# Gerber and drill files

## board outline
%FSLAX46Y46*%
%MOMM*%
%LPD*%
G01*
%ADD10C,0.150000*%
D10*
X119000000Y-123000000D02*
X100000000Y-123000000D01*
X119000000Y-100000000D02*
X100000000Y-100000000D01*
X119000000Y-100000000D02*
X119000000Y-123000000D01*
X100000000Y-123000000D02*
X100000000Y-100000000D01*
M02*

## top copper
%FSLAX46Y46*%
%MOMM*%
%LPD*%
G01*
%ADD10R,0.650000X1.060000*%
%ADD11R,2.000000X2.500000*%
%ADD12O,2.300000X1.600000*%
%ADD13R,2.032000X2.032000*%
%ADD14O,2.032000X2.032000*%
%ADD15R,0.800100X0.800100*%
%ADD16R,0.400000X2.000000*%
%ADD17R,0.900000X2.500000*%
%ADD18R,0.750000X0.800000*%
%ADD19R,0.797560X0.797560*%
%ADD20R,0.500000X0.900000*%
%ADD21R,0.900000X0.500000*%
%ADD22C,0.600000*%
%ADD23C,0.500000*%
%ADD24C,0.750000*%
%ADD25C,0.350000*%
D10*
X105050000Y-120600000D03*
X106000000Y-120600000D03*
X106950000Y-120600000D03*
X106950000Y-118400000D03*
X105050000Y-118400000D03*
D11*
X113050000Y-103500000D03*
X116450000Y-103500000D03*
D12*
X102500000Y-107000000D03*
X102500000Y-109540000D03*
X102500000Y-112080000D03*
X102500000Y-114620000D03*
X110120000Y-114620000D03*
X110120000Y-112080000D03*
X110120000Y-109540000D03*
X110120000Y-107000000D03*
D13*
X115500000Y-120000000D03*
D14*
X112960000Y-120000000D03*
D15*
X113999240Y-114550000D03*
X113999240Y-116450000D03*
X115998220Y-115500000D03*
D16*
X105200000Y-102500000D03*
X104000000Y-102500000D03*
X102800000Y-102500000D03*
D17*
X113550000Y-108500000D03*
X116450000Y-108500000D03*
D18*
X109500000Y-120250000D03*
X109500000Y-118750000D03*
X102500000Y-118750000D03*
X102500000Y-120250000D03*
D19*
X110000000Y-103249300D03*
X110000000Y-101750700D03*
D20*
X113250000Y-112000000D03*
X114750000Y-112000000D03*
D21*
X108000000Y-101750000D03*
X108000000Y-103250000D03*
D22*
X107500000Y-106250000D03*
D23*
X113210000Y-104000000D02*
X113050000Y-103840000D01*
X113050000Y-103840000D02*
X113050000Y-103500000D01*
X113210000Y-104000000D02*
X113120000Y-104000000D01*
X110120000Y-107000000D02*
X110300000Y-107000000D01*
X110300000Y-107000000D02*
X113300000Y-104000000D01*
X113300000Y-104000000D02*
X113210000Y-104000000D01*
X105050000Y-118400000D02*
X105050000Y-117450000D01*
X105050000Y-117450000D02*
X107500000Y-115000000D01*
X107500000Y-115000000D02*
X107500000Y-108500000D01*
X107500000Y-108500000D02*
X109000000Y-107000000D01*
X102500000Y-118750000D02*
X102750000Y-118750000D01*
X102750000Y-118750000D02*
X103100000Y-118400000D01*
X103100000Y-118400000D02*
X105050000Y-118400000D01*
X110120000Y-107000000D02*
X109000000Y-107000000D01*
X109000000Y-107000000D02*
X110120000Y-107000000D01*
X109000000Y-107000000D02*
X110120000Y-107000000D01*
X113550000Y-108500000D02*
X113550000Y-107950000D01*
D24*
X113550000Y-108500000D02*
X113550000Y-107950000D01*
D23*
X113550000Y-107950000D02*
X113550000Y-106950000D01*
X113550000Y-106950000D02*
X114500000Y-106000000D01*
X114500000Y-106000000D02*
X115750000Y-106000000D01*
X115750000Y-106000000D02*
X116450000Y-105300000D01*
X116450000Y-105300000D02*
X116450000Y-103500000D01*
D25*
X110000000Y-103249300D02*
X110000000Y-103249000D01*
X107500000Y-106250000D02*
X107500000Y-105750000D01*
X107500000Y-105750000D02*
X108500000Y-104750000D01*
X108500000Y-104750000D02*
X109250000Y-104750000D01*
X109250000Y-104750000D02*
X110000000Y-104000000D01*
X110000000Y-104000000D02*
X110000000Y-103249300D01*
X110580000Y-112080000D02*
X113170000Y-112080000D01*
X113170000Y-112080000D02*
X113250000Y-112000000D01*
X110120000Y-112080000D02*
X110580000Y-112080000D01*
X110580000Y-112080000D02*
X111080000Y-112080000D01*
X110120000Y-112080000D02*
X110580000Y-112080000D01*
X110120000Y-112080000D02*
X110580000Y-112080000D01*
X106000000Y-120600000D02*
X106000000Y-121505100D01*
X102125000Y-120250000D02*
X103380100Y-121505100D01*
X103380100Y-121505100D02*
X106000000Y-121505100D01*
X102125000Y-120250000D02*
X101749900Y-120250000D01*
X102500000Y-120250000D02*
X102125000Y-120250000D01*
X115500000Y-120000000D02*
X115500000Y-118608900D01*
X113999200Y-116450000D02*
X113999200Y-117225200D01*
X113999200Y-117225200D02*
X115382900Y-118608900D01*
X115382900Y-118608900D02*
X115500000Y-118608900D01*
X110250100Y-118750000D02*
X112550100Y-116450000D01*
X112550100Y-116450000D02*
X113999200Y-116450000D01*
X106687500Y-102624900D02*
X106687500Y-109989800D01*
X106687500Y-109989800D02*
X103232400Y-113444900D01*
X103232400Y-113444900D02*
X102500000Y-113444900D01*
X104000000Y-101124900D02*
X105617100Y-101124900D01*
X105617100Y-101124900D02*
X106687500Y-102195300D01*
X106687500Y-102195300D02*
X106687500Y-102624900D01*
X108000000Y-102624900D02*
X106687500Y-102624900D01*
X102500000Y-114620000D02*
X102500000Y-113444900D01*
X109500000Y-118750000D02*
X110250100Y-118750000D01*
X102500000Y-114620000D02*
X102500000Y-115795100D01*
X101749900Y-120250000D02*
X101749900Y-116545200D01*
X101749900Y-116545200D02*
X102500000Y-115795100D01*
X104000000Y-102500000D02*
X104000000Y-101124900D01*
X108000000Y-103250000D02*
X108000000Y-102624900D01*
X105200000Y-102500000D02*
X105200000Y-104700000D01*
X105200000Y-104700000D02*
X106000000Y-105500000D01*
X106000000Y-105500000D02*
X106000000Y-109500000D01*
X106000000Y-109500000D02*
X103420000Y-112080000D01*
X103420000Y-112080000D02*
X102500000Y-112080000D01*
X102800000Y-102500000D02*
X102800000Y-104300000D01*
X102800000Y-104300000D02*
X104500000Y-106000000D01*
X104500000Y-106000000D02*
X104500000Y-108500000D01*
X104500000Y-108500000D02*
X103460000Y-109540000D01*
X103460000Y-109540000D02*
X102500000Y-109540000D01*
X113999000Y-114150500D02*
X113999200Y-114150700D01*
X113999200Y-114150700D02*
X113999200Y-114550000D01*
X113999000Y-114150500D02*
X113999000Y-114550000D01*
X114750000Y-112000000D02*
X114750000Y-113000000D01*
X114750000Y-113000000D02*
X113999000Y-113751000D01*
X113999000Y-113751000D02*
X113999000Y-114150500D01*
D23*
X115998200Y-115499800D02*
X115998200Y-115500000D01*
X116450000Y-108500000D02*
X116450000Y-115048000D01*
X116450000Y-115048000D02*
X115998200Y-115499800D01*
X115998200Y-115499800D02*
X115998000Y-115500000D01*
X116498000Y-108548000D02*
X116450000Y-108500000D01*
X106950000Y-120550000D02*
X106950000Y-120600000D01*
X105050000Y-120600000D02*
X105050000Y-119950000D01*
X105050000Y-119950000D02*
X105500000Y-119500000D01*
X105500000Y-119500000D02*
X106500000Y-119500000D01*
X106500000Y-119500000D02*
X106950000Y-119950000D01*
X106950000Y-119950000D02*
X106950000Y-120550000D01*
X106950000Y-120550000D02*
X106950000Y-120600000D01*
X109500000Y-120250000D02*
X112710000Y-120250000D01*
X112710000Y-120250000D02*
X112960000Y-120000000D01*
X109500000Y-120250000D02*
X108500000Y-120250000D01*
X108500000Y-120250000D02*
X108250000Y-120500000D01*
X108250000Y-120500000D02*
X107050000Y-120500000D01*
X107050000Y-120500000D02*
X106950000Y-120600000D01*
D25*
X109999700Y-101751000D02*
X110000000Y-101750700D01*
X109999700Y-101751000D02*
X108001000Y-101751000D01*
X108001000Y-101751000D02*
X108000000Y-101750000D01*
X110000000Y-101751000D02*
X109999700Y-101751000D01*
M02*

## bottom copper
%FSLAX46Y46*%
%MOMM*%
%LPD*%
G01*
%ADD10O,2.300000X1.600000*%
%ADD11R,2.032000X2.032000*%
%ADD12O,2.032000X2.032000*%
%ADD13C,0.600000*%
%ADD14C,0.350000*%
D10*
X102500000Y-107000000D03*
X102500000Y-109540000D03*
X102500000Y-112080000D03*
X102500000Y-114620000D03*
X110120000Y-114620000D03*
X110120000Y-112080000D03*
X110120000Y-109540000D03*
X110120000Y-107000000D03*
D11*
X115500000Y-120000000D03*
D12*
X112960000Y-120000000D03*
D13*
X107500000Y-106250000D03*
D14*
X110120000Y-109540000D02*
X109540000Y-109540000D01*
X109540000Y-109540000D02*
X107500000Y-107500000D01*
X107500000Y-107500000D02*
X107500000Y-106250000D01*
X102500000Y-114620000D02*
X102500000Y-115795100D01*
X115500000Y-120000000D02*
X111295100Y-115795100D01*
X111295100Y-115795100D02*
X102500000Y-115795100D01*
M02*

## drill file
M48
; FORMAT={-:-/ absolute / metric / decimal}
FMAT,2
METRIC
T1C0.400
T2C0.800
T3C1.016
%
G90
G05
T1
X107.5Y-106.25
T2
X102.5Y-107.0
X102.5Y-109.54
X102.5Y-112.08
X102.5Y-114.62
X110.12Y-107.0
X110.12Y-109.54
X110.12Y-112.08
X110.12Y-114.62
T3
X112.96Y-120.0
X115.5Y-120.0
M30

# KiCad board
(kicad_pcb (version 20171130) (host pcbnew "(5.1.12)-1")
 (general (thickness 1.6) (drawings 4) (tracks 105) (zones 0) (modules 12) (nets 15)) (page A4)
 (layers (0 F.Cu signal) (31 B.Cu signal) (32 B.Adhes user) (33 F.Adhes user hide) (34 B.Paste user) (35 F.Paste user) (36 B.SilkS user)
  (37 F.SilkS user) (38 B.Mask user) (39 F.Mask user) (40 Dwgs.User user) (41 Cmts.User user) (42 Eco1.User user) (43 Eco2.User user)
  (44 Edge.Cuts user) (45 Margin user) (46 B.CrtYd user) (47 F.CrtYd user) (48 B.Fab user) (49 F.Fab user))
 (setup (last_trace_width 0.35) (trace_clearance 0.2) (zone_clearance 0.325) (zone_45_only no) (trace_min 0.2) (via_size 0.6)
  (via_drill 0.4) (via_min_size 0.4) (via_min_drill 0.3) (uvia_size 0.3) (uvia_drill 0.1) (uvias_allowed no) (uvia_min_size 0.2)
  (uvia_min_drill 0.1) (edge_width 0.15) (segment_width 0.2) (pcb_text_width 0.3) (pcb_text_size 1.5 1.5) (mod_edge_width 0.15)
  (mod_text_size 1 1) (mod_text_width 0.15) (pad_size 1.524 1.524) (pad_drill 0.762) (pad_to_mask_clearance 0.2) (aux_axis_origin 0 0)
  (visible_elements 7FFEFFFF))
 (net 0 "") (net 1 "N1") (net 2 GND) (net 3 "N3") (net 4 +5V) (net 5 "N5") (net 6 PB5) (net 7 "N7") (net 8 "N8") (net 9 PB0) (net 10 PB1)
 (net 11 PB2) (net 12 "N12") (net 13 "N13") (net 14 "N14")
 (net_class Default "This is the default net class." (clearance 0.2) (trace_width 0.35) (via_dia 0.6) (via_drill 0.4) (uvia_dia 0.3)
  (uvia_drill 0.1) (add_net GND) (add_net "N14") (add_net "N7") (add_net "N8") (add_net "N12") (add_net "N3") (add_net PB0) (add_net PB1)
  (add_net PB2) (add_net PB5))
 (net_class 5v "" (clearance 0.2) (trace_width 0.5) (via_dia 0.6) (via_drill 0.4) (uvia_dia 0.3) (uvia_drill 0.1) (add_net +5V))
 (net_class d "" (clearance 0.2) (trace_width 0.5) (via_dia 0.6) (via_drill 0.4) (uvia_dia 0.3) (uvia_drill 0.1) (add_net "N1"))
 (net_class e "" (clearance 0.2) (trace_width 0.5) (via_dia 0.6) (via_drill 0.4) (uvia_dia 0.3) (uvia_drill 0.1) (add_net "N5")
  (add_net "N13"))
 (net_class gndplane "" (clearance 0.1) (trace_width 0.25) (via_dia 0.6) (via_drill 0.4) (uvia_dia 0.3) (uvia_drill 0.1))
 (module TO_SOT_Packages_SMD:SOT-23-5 (layer F.Cu) (at 106 119.5 90)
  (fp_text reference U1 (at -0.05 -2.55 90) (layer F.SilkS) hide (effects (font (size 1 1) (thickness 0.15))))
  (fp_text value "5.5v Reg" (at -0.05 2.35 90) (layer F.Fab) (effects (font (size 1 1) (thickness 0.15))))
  (pad 1 smd rect (at -1.1 -0.95 90) (size 1.06 0.65) (layers F.Cu F.Paste F.Mask) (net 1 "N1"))
  (pad 2 smd rect (at -1.1 0 90) (size 1.06 0.65) (layers F.Cu F.Paste F.Mask) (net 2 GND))
  (pad 3 smd rect (at -1.1 0.95 90) (size 1.06 0.65) (layers F.Cu F.Paste F.Mask) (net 1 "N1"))
  (pad 4 smd rect (at 1.1 0.95 90) (size 1.06 0.65) (layers F.Cu F.Paste F.Mask) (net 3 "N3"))
  (pad 5 smd rect (at 1.1 -0.95 90) (size 1.06 0.65) (layers F.Cu F.Paste F.Mask) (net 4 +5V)))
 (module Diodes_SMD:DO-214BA (layer F.Cu) (at 114.75 103.5 180)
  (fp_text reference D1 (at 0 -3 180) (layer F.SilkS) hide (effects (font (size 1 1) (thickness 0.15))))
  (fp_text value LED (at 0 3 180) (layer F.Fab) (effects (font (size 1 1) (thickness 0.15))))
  (pad 2 smd rect (at 1.7 0 180) (size 2 2.5) (layers F.Cu F.Paste F.Mask) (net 4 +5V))
  (pad 1 smd rect (at -1.7 0 180) (size 2 2.5) (layers F.Cu F.Paste F.Mask) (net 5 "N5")))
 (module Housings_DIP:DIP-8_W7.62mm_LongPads (layer F.Cu) (at 102.5 107)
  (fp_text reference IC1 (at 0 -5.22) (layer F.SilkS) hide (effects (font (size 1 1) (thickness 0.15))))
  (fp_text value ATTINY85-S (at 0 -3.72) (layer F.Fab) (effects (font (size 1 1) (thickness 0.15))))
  (pad 1 thru_hole oval (at 0 0) (size 2.3 1.6) (drill 0.8) (layers *.Cu *.Mask F.SilkS) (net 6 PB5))
  (pad 2 thru_hole oval (at 0 2.54) (size 2.3 1.6) (drill 0.8) (layers *.Cu *.Mask F.SilkS) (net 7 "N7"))
  (pad 3 thru_hole oval (at 0 5.08) (size 2.3 1.6) (drill 0.8) (layers *.Cu *.Mask F.SilkS) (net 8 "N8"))
  (pad 4 thru_hole oval (at 0 7.62) (size 2.3 1.6) (drill 0.8) (layers *.Cu *.Mask F.SilkS) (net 2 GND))
  (pad 5 thru_hole oval (at 7.62 7.62) (size 2.3 1.6) (drill 0.8) (layers *.Cu *.Mask F.SilkS) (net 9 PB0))
  (pad 6 thru_hole oval (at 7.62 5.08) (size 2.3 1.6) (drill 0.8) (layers *.Cu *.Mask F.SilkS) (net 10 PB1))
  (pad 7 thru_hole oval (at 7.62 2.54) (size 2.3 1.6) (drill 0.8) (layers *.Cu *.Mask F.SilkS) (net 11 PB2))
  (pad 8 thru_hole oval (at 7.62 0) (size 2.3 1.6) (drill 0.8) (layers *.Cu *.Mask F.SilkS) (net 4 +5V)))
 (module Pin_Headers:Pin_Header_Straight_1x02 (layer F.Cu) (at 115.5 120 270)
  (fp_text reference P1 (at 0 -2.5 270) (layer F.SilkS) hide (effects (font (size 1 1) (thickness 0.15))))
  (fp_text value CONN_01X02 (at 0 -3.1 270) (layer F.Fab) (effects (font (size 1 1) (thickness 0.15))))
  (pad 1 thru_hole rect (at 0 0 270) (size 2.032 2.032) (drill 1.016) (layers *.Cu *.Mask F.SilkS) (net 2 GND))
  (pad 2 thru_hole oval (at 0 2.54 270) (size 2.032 2.032) (drill 1.016) (layers *.Cu *.Mask F.SilkS) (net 1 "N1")))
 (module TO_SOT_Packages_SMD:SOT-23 (layer F.Cu) (at 115 115.5 270)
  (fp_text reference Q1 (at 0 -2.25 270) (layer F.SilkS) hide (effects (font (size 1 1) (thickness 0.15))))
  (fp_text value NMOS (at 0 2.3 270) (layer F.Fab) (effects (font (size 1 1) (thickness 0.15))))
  (pad 1 smd rect (at -0.95 1.00076 270) (size 0.8001 0.8001) (layers F.Cu F.Paste F.Mask) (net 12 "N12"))
  (pad 2 smd rect (at 0.95 1.00076 270) (size 0.8001 0.8001) (layers F.Cu F.Paste F.Mask) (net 2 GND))
  (pad 3 smd rect (at 0 -0.99822 270) (size 0.8001 0.8001) (layers F.Cu F.Paste F.Mask) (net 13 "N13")))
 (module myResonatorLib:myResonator (layer F.Cu) (at 104 102.5)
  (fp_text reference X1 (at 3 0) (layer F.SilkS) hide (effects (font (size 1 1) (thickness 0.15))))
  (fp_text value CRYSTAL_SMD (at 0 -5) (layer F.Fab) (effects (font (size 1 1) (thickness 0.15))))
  (pad 2 smd rect (at 1.2 0) (size 0.4 2) (layers F.Cu F.Paste F.Mask) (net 8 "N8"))
  (pad 3 smd rect (at 0 0) (size 0.4 2) (layers F.Cu F.Paste F.Mask) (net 2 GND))
  (pad 1 smd rect (at -1.2 0) (size 0.4 2) (layers F.Cu F.Paste F.Mask) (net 7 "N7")))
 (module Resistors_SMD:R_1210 (layer F.Cu) (at 115 108.5)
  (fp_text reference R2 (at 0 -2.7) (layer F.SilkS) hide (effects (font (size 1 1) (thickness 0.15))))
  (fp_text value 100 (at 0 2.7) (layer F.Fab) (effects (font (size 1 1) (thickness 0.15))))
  (pad 1 smd rect (at -1.45 0) (size 0.9 2.5) (layers F.Cu F.Paste F.Mask) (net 5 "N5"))
  (pad 2 smd rect (at 1.45 0) (size 0.9 2.5) (layers F.Cu F.Paste F.Mask) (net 13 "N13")))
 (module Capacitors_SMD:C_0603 (layer F.Cu) (at 109.5 119.5 90)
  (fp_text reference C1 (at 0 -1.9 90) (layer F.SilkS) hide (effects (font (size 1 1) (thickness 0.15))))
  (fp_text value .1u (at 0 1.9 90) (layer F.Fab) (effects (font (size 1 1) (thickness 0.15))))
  (pad 1 smd rect (at -0.75 0 90) (size 0.8 0.75) (layers F.Cu F.Paste F.Mask) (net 1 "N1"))
  (pad 2 smd rect (at 0.75 0 90) (size 0.8 0.75) (layers F.Cu F.Paste F.Mask) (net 2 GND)))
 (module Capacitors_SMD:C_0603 (layer F.Cu) (at 102.5 119.5 270)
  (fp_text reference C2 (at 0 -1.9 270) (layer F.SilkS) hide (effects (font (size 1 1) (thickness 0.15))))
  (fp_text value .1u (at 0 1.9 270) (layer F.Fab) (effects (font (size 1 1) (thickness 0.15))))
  (pad 1 smd rect (at -0.75 0 270) (size 0.8 0.75) (layers F.Cu F.Paste F.Mask) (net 4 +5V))
  (pad 2 smd rect (at 0.75 0 270) (size 0.8 0.75) (layers F.Cu F.Paste F.Mask) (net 2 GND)))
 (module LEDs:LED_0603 (layer F.Cu) (at 110 102.5 270)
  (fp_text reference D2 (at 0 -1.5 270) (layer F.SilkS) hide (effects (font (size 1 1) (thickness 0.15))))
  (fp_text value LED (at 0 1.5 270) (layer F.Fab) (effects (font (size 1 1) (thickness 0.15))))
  (pad 2 smd rect (at 0.7493 0 90) (size 0.79756 0.79756) (layers F.Cu F.Paste F.Mask) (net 11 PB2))
  (pad 1 smd rect (at -0.7493 0 90) (size 0.79756 0.79756) (layers F.Cu F.Paste F.Mask) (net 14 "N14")))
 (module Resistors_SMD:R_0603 (layer F.Cu) (at 114 112)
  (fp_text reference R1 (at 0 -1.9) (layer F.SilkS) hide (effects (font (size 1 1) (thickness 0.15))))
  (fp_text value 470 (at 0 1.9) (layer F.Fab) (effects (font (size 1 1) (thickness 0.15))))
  (pad 1 smd rect (at -0.75 0) (size 0.5 0.9) (layers F.Cu F.Paste F.Mask) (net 10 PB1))
  (pad 2 smd rect (at 0.75 0) (size 0.5 0.9) (layers F.Cu F.Paste F.Mask) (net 12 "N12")))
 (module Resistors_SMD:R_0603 (layer F.Cu) (at 108 102.5 270)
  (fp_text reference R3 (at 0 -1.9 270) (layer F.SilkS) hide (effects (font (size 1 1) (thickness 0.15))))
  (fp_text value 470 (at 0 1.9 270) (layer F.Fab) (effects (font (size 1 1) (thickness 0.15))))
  (pad 1 smd rect (at -0.75 0 270) (size 0.5 0.9) (layers F.Cu F.Paste F.Mask) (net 14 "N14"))
  (pad 2 smd rect (at 0.75 0 270) (size 0.5 0.9) (layers F.Cu F.Paste F.Mask) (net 2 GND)))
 (gr_line (start 119 123) (end 100 123) (angle 90) (layer Edge.Cuts) (width 0.15))
 (gr_line (start 119 100) (end 100 100) (angle 90) (layer Edge.Cuts) (width 0.15))
 (gr_line (start 119 100) (end 119 123) (angle 90) (layer Edge.Cuts) (width 0.15))
 (gr_line (start 100 123) (end 100 100) (angle 90) (layer Edge.Cuts) (width 0.15))
 (segment (start 113.21 104) (end 113.05 103.84) (width 0.5) (layer F.Cu) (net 4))
 (segment (start 113.05 103.84) (end 113.05 103.5) (width 0.5) (layer F.Cu) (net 4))
 (segment (start 113.21 104) (end 113.12 104) (width 0.5) (layer F.Cu) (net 4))
 (segment (start 110.12 107) (end 110.3 107) (width 0.5) (layer F.Cu) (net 4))
 (segment (start 110.3 107) (end 113.3 104) (width 0.5) (layer F.Cu) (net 4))
 (segment (start 113.3 104) (end 113.21 104) (width 0.5) (layer F.Cu) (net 4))
 (segment (start 105.05 118.4) (end 105.05 117.45) (width 0.5) (layer F.Cu) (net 4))
 (segment (start 105.05 117.45) (end 107.5 115) (width 0.5) (layer F.Cu) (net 4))
 (segment (start 107.5 115) (end 107.5 108.5) (width 0.5) (layer F.Cu) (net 4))
 (segment (start 107.5 108.5) (end 109 107) (width 0.5) (layer F.Cu) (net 4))
 (segment (start 102.5 118.75) (end 102.75 118.75) (width 0.5) (layer F.Cu) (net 4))
 (segment (start 102.75 118.75) (end 103.1 118.4) (width 0.5) (layer F.Cu) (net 4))
 (segment (start 103.1 118.4) (end 105.05 118.4) (width 0.5) (layer F.Cu) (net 4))
 (segment (start 110.12 107) (end 109 107) (width 0.5) (layer F.Cu) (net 4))
 (segment (start 109 107) (end 110.12 107) (width 0.5) (layer F.Cu) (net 4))
 (segment (start 109 107) (end 110.12 107) (width 0.5) (layer F.Cu) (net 4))
 (segment (start 113.55 108.5) (end 113.55 107.95) (width 0.5) (layer F.Cu) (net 5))
 (segment (start 113.55 108.5) (end 113.55 107.95) (width 0.75) (layer F.Cu) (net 5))
 (segment (start 113.55 107.95) (end 113.55 106.95) (width 0.5) (layer F.Cu) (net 5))
 (segment (start 113.55 106.95) (end 114.5 106) (width 0.5) (layer F.Cu) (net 5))
 (segment (start 114.5 106) (end 115.75 106) (width 0.5) (layer F.Cu) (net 5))
 (segment (start 115.75 106) (end 116.45 105.3) (width 0.5) (layer F.Cu) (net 5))
 (segment (start 116.45 105.3) (end 116.45 103.5) (width 0.5) (layer F.Cu) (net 5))
 (segment (start 110 103.2493) (end 110 103.249) (width 0.35) (layer F.Cu) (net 11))
 (segment (start 107.5 106.25) (end 107.5 105.75) (width 0.35) (layer F.Cu) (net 11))
 (segment (start 107.5 105.75) (end 108.5 104.75) (width 0.35) (layer F.Cu) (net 11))
 (segment (start 108.5 104.75) (end 109.25 104.75) (width 0.35) (layer F.Cu) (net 11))
 (segment (start 109.25 104.75) (end 110 104) (width 0.35) (layer F.Cu) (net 11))
 (segment (start 110 104) (end 110 103.2493) (width 0.35) (layer F.Cu) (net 11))
 (segment (start 110.12 109.54) (end 109.54 109.54) (width 0.35) (layer B.Cu) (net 11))
 (segment (start 109.54 109.54) (end 107.5 107.5) (width 0.35) (layer B.Cu) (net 11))
 (segment (start 107.5 107.5) (end 107.5 106.25) (width 0.35) (layer B.Cu) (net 11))
 (via (at 107.5 106.25) (size 0.6) (layers F.Cu B.Cu) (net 11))
 (segment (start 110.58 112.08) (end 113.17 112.08) (width 0.35) (layer F.Cu) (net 10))
 (segment (start 113.17 112.08) (end 113.25 112) (width 0.35) (layer F.Cu) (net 10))
 (segment (start 110.12 112.08) (end 110.58 112.08) (width 0.35) (layer F.Cu) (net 10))
 (segment (start 110.58 112.08) (end 111.08 112.08) (width 0.35) (layer F.Cu) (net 10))
 (segment (start 110.12 112.08) (end 110.58 112.08) (width 0.35) (layer F.Cu) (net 10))
 (segment (start 110.12 112.08) (end 110.58 112.08) (width 0.35) (layer F.Cu) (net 10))
 (segment (start 106 120.6) (end 106 121.5051) (width 0.35) (layer F.Cu) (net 2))
 (segment (start 102.125 120.25) (end 103.3801 121.5051) (width 0.35) (layer F.Cu) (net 2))
 (segment (start 103.3801 121.5051) (end 106 121.5051) (width 0.35) (layer F.Cu) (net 2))
 (segment (start 102.125 120.25) (end 101.7499 120.25) (width 0.35) (layer F.Cu) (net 2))
 (segment (start 102.5 120.25) (end 102.125 120.25) (width 0.35) (layer F.Cu) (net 2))
 (segment (start 102.5 114.62) (end 102.5 115.7951) (width 0.35) (layer B.Cu) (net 2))
 (segment (start 115.5 120) (end 111.2951 115.7951) (width 0.35) (layer B.Cu) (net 2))
 (segment (start 111.2951 115.7951) (end 102.5 115.7951) (width 0.35) (layer B.Cu) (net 2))
 (segment (start 115.5 120) (end 115.5 118.6089) (width 0.35) (layer F.Cu) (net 2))
 (segment (start 113.9992 116.45) (end 113.9992 117.2252) (width 0.35) (layer F.Cu) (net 2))
 (segment (start 113.9992 117.2252) (end 115.3829 118.6089) (width 0.35) (layer F.Cu) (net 2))
 (segment (start 115.3829 118.6089) (end 115.5 118.6089) (width 0.35) (layer F.Cu) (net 2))
 (segment (start 110.2501 118.75) (end 112.5501 116.45) (width 0.35) (layer F.Cu) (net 2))
 (segment (start 112.5501 116.45) (end 113.9992 116.45) (width 0.35) (layer F.Cu) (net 2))
 (segment (start 106.6875 102.6249) (end 106.6875 109.9898) (width 0.35) (layer F.Cu) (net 2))
 (segment (start 106.6875 109.9898) (end 103.2324 113.4449) (width 0.35) (layer F.Cu) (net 2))
 (segment (start 103.2324 113.4449) (end 102.5 113.4449) (width 0.35) (layer F.Cu) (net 2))
 (segment (start 104 101.1249) (end 105.6171 101.1249) (width 0.35) (layer F.Cu) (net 2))
 (segment (start 105.6171 101.1249) (end 106.6875 102.1953) (width 0.35) (layer F.Cu) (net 2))
 (segment (start 106.6875 102.1953) (end 106.6875 102.6249) (width 0.35) (layer F.Cu) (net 2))
 (segment (start 108 102.6249) (end 106.6875 102.6249) (width 0.35) (layer F.Cu) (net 2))
 (segment (start 102.5 114.62) (end 102.5 113.4449) (width 0.35) (layer F.Cu) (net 2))
 (segment (start 109.5 118.75) (end 110.2501 118.75) (width 0.35) (layer F.Cu) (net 2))
 (segment (start 102.5 114.62) (end 102.5 115.7951) (width 0.35) (layer F.Cu) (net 2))
 (segment (start 101.7499 120.25) (end 101.7499 116.5452) (width 0.35) (layer F.Cu) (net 2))
 (segment (start 101.7499 116.5452) (end 102.5 115.7951) (width 0.35) (layer F.Cu) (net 2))
 (segment (start 104 102.5) (end 104 101.1249) (width 0.35) (layer F.Cu) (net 2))
 (segment (start 108 103.25) (end 108 102.6249) (width 0.35) (layer F.Cu) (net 2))
 (segment (start 105.2 102.5) (end 105.2 104.7) (width 0.35) (layer F.Cu) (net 8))
 (segment (start 105.2 104.7) (end 106 105.5) (width 0.35) (layer F.Cu) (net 8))
 (segment (start 106 105.5) (end 106 109.5) (width 0.35) (layer F.Cu) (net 8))
 (segment (start 106 109.5) (end 103.42 112.08) (width 0.35) (layer F.Cu) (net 8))
 (segment (start 103.42 112.08) (end 102.5 112.08) (width 0.35) (layer F.Cu) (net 8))
 (segment (start 102.8 102.5) (end 102.8 104.3) (width 0.35) (layer F.Cu) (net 7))
 (segment (start 102.8 104.3) (end 104.5 106) (width 0.35) (layer F.Cu) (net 7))
 (segment (start 104.5 106) (end 104.5 108.5) (width 0.35) (layer F.Cu) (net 7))
 (segment (start 104.5 108.5) (end 103.46 109.54) (width 0.35) (layer F.Cu) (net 7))
 (segment (start 103.46 109.54) (end 102.5 109.54) (width 0.35) (layer F.Cu) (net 7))
 (segment (start 113.999 114.1505) (end 113.9992 114.1507) (width 0.35) (layer F.Cu) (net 12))
 (segment (start 113.9992 114.1507) (end 113.9992 114.55) (width 0.35) (layer F.Cu) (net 12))
 (segment (start 113.999 114.1505) (end 113.999 114.55) (width 0.35) (layer F.Cu) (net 12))
 (segment (start 114.75 112) (end 114.75 113) (width 0.35) (layer F.Cu) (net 12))
 (segment (start 114.75 113) (end 113.999 113.751) (width 0.35) (layer F.Cu) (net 12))
 (segment (start 113.999 113.751) (end 113.999 114.1505) (width 0.35) (layer F.Cu) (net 12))
 (segment (start 115.9982 115.4998) (end 115.9982 115.5) (width 0.5) (layer F.Cu) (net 13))
 (segment (start 116.45 108.5) (end 116.45 115.048) (width 0.5) (layer F.Cu) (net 13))
 (segment (start 116.45 115.048) (end 115.9982 115.4998) (width 0.5) (layer F.Cu) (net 13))
 (segment (start 115.9982 115.4998) (end 115.998 115.5) (width 0.5) (layer F.Cu) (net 13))
 (segment (start 116.498 108.548) (end 116.45 108.5) (width 0.5) (layer F.Cu) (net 13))
 (segment (start 106.95 120.55) (end 106.95 120.6) (width 0.5) (layer F.Cu) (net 1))
 (segment (start 105.05 120.6) (end 105.05 119.95) (width 0.5) (layer F.Cu) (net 1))
 (segment (start 105.05 119.95) (end 105.5 119.5) (width 0.5) (layer F.Cu) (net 1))
 (segment (start 105.5 119.5) (end 106.5 119.5) (width 0.5) (layer F.Cu) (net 1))
 (segment (start 106.5 119.5) (end 106.95 119.95) (width 0.5) (layer F.Cu) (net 1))
 (segment (start 106.95 119.95) (end 106.95 120.55) (width 0.5) (layer F.Cu) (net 1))
 (segment (start 106.95 120.55) (end 106.95 120.6) (width 0.5) (layer F.Cu) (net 1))
 (segment (start 109.5 120.25) (end 112.71 120.25) (width 0.5) (layer F.Cu) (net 1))
 (segment (start 112.71 120.25) (end 112.96 120) (width 0.5) (layer F.Cu) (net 1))
 (segment (start 109.5 120.25) (end 108.5 120.25) (width 0.5) (layer F.Cu) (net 1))
 (segment (start 108.5 120.25) (end 108.25 120.5) (width 0.5) (layer F.Cu) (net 1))
 (segment (start 108.25 120.5) (end 107.05 120.5) (width 0.5) (layer F.Cu) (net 1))
 (segment (start 107.05 120.5) (end 106.95 120.6) (width 0.5) (layer F.Cu) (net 1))
 (segment (start 109.9997 101.751) (end 110 101.7507) (width 0.35) (layer F.Cu) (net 14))
 (segment (start 109.9997 101.751) (end 108.001 101.751) (width 0.35) (layer F.Cu) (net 14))
 (segment (start 108.001 101.751) (end 108 101.75) (width 0.35) (layer F.Cu) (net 14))
 (segment (start 110 101.751) (end 109.9997 101.751) (width 0.35) (layer F.Cu) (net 14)))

